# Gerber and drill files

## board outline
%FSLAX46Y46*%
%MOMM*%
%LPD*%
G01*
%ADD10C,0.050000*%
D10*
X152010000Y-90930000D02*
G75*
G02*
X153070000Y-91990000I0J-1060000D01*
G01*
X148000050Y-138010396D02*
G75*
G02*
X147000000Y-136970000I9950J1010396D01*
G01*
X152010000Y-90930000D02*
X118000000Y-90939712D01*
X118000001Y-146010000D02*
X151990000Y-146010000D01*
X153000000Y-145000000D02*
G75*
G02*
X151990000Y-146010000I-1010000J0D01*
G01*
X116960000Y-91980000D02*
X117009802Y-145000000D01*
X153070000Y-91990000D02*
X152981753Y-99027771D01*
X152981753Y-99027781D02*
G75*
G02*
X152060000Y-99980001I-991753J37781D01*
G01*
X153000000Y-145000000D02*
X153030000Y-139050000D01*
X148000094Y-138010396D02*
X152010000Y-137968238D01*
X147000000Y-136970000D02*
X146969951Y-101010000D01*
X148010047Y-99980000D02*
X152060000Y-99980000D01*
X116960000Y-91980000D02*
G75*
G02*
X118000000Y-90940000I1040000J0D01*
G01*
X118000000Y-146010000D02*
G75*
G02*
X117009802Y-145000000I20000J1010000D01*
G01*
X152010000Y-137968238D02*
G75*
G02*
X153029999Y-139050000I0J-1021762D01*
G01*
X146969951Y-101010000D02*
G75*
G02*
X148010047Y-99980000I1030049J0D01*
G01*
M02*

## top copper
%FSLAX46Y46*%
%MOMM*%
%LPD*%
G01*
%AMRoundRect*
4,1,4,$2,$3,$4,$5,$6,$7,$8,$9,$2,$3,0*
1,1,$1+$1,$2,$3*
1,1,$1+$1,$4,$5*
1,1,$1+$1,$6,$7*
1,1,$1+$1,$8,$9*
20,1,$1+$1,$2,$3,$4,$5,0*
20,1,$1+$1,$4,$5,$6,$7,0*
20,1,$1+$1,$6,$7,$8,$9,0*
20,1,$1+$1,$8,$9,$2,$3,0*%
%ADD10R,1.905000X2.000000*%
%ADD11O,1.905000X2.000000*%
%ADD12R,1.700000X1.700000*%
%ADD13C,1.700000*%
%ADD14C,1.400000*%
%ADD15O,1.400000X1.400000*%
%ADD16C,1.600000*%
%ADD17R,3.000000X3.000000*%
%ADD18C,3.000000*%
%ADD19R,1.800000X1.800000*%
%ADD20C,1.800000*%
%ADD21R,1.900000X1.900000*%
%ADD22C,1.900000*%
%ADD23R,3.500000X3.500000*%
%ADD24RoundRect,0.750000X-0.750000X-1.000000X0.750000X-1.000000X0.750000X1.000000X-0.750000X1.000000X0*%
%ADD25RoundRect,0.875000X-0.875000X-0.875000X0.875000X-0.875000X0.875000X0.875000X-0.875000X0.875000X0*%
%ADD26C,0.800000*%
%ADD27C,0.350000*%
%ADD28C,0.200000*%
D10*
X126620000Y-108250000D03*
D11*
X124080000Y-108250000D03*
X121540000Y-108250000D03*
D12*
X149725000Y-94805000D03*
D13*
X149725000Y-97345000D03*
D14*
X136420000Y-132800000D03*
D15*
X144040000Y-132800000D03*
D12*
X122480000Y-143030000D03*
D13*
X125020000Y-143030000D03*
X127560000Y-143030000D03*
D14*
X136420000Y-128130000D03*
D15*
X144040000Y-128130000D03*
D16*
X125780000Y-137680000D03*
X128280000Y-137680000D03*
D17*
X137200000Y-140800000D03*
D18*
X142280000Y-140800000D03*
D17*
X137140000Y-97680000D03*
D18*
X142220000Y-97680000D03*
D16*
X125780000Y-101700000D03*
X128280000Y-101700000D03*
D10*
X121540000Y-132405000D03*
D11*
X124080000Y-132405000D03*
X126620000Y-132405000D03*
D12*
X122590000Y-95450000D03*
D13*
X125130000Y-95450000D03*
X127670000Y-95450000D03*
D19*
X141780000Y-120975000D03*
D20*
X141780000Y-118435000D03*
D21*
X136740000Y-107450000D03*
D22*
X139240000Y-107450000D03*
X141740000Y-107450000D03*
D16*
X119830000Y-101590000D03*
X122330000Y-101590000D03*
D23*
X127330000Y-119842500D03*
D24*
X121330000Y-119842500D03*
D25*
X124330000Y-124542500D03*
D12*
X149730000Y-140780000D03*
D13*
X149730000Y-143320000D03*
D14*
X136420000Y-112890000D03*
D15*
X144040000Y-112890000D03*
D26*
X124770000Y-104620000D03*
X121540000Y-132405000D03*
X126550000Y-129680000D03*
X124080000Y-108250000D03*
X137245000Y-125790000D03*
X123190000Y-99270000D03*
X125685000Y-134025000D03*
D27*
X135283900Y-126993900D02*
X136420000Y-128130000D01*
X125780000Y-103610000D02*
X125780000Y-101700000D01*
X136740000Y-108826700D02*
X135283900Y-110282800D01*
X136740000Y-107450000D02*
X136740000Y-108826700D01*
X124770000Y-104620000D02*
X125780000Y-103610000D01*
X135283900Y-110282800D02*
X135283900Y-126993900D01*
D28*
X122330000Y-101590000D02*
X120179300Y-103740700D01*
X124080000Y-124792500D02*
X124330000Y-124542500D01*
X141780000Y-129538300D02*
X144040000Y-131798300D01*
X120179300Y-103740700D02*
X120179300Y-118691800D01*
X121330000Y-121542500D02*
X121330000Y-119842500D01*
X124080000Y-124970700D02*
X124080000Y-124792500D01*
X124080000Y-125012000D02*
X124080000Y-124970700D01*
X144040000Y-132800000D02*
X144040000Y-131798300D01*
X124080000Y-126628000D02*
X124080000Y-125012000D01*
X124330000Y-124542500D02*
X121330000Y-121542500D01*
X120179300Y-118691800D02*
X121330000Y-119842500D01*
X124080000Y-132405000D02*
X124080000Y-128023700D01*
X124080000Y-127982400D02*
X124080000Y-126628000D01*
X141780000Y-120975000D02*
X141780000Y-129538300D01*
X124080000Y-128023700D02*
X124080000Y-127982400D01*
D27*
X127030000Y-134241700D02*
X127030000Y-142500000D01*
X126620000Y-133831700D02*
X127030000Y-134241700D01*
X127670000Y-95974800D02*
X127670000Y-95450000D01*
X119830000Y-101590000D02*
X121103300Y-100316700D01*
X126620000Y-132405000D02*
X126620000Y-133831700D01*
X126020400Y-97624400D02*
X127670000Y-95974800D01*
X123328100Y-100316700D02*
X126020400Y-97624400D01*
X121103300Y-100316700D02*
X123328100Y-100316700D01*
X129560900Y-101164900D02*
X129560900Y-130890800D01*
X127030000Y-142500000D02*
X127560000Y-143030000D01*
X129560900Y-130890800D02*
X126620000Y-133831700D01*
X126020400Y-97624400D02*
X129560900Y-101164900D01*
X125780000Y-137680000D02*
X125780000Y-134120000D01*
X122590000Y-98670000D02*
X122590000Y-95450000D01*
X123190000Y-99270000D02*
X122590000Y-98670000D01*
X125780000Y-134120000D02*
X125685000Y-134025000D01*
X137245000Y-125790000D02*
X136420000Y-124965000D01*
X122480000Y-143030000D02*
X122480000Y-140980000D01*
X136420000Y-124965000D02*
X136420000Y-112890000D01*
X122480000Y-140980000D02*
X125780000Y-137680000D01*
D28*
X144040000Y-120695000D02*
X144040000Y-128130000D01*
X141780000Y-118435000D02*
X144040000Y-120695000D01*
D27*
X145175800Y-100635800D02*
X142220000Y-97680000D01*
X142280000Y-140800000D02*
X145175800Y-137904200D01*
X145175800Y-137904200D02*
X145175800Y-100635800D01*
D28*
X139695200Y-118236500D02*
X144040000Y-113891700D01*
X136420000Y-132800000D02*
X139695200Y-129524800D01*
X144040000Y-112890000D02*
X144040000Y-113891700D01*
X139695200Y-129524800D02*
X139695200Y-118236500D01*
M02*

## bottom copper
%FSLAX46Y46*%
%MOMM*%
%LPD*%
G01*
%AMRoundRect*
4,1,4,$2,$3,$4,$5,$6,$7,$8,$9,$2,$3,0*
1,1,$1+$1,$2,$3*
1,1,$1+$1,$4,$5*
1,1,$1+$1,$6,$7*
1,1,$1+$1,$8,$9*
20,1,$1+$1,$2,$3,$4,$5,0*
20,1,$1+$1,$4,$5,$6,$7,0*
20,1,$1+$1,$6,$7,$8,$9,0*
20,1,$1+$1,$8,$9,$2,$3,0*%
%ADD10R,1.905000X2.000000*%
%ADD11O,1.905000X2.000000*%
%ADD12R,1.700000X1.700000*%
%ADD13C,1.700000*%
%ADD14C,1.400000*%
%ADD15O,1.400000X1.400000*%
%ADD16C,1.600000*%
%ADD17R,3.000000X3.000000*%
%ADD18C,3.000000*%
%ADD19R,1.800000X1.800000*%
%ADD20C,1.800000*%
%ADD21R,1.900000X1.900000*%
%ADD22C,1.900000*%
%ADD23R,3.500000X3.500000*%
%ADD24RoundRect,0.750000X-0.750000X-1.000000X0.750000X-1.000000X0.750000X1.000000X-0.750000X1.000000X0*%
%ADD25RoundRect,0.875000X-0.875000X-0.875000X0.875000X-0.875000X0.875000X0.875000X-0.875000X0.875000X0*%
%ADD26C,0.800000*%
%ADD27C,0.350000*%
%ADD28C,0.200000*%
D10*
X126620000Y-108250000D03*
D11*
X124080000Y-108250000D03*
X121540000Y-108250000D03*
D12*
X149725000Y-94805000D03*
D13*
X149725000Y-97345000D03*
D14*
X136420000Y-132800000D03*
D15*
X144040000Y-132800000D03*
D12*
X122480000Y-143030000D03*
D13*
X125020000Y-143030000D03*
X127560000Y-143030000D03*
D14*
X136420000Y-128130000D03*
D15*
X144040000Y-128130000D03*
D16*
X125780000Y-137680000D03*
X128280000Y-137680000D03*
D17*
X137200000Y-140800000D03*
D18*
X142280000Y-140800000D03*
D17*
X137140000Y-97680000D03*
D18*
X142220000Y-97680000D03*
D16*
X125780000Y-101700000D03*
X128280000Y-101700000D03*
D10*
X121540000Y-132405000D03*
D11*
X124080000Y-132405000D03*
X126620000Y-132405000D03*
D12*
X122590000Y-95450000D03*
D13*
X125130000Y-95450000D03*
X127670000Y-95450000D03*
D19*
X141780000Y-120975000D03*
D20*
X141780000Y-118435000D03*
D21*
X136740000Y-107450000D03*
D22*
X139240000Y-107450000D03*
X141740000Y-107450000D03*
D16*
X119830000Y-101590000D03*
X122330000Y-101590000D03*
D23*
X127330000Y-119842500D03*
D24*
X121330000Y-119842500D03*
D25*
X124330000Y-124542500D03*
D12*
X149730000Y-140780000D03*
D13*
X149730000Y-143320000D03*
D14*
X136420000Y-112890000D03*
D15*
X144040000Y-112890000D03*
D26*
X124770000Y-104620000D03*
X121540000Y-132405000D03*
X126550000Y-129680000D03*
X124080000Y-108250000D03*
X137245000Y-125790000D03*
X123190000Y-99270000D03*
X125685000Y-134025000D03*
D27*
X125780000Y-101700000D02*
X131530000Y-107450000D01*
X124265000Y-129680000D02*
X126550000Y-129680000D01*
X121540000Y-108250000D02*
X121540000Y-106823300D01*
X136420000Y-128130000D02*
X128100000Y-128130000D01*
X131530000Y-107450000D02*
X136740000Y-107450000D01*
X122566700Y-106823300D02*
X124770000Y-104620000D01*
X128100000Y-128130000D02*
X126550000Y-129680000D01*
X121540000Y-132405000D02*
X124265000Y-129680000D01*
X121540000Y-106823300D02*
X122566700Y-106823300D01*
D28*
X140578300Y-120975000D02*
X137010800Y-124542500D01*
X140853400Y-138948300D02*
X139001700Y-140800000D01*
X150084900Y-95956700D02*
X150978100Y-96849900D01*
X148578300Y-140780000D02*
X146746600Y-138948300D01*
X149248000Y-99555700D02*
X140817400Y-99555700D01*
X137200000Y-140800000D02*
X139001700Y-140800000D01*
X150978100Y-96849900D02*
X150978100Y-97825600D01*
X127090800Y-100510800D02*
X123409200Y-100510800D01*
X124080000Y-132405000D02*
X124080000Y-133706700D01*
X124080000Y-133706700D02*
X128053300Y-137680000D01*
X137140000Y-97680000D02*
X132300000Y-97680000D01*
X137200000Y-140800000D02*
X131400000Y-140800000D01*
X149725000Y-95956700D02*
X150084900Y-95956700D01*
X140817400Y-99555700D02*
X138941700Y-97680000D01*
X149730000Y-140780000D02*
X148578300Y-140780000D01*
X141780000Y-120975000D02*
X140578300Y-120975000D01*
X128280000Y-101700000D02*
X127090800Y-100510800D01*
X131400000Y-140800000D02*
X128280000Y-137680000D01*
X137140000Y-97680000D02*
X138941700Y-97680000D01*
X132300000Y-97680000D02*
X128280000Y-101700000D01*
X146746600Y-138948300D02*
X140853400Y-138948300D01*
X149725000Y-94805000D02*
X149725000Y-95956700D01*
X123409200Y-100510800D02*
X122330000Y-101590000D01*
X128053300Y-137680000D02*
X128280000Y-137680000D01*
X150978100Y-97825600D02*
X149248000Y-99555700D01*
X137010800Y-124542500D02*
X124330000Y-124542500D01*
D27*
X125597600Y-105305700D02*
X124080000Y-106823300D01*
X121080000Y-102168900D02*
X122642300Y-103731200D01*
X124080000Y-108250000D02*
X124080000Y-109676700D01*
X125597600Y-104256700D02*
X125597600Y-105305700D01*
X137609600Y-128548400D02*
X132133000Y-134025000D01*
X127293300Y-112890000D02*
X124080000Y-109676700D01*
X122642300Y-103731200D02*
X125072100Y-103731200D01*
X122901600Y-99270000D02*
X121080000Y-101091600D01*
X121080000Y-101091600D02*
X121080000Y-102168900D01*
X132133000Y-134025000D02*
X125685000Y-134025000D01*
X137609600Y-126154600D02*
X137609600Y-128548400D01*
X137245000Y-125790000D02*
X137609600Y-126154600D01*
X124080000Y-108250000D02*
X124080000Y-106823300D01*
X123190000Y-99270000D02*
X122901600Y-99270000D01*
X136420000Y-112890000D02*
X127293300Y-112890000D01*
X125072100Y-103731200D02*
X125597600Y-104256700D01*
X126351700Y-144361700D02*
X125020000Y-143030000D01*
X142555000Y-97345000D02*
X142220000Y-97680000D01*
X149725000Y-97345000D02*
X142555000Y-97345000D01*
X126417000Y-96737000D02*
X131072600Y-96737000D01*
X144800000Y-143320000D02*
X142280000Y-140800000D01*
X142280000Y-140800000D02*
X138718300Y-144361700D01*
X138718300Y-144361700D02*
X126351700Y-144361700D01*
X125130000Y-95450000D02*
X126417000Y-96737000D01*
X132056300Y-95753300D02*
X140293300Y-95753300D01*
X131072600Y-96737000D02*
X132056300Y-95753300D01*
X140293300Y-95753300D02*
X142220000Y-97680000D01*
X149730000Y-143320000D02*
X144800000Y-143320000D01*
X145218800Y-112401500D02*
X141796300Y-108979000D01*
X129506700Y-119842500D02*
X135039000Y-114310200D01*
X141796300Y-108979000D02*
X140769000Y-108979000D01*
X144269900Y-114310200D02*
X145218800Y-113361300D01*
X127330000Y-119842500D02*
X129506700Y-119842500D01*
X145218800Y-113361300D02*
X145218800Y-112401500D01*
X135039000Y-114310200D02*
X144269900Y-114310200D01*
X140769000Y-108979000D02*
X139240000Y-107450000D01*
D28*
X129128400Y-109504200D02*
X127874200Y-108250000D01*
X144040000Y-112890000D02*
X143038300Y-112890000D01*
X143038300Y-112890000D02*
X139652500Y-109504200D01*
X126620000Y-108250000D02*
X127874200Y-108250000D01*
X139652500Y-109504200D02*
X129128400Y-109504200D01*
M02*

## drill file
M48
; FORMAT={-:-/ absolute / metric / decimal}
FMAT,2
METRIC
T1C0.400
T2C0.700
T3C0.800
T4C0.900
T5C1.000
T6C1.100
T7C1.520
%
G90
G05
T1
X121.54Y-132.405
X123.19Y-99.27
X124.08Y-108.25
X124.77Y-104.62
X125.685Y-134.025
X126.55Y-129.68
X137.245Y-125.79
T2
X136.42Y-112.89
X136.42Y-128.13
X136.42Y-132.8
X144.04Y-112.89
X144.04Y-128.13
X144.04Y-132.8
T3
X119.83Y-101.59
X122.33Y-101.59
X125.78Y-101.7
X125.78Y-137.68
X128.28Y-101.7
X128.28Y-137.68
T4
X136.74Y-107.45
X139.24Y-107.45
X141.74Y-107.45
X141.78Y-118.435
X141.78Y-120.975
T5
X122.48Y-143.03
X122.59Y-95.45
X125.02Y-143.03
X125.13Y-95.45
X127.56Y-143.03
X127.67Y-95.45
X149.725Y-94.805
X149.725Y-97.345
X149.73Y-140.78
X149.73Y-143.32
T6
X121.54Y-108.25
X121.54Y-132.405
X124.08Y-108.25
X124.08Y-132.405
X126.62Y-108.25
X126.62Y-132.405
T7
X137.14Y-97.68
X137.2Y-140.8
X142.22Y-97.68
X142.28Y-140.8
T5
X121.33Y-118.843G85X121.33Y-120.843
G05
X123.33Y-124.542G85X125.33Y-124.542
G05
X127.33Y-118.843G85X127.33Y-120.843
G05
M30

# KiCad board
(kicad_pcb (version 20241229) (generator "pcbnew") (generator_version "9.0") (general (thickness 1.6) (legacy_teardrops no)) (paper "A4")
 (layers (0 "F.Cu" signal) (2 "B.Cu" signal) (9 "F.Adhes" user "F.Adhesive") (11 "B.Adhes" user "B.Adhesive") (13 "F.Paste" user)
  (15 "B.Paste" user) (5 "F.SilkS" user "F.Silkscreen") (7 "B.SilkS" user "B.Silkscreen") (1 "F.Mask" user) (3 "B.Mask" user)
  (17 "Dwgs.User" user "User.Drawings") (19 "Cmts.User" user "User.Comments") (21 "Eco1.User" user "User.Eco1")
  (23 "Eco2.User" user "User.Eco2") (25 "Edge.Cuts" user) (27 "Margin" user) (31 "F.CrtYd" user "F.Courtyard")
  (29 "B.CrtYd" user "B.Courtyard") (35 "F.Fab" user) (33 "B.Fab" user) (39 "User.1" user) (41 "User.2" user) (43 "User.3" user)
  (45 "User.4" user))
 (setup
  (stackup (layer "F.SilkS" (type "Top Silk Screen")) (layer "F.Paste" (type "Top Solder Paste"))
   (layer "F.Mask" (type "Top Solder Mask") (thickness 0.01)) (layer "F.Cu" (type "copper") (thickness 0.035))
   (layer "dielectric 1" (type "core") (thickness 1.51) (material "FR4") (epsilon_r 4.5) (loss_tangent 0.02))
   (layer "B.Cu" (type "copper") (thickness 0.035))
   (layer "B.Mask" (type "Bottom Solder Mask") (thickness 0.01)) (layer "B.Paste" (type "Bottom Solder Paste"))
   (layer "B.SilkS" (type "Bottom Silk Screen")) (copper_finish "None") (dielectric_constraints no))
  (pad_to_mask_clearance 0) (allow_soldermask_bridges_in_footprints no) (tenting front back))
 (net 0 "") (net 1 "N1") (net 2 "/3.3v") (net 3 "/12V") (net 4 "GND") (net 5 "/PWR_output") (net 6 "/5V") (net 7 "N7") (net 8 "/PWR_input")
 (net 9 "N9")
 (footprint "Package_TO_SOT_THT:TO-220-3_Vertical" (layer "F.Cu") (at 126.62 108.25 180)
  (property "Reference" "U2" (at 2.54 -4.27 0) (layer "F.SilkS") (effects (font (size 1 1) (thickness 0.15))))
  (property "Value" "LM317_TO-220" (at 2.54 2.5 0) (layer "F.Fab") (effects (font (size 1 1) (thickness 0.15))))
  (pad "1" thru_hole rect (at 0 0 180) (size 1.905 2) (drill 1.1) (layers "*.Cu" "*.Mask") (remove_unused_layers no) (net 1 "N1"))
  (pad "2" thru_hole oval (at 2.54 0 180) (size 1.905 2) (drill 1.1) (layers "*.Cu" "*.Mask") (remove_unused_layers no) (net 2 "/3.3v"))
  (pad "3" thru_hole oval (at 5.08 0 180) (size 1.905 2) (drill 1.1) (layers "*.Cu" "*.Mask") (remove_unused_layers no) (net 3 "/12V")))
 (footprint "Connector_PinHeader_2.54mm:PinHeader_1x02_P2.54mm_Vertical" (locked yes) (layer "F.Cu") (at 149.725 94.805)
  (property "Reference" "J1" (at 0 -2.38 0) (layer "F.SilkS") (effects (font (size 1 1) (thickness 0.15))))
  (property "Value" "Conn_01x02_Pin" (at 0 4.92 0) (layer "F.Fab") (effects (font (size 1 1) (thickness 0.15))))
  (pad "1" thru_hole rect (at 0 0) (size 1.7 1.7) (drill 1) (layers "*.Cu" "*.Mask") (remove_unused_layers no) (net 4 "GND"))
  (pad "2" thru_hole circle (at 0 2.54) (size 1.7 1.7) (drill 1) (layers "*.Cu" "*.Mask") (remove_unused_layers no) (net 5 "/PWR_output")))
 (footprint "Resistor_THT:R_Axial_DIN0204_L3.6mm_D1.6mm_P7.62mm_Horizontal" (layer "F.Cu") (at 136.42 132.8)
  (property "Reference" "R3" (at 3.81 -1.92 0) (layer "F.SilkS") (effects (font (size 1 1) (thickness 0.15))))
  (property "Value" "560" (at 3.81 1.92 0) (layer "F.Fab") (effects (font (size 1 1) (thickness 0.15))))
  (pad "1" thru_hole circle (at 0 0) (size 1.4 1.4) (drill 0.7) (layers "*.Cu" "*.Mask") (remove_unused_layers no) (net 1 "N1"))
  (pad "2" thru_hole oval (at 7.62 0) (size 1.4 1.4) (drill 0.7) (layers "*.Cu" "*.Mask") (remove_unused_layers no) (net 4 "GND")))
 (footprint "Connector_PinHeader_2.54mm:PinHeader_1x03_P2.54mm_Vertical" (layer "F.Cu") (at 122.48 143.03 90)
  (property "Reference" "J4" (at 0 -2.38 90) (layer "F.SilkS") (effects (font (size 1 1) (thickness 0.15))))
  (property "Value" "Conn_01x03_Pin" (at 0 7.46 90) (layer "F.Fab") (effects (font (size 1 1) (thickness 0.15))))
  (pad "1" thru_hole rect (at 0 0 90) (size 1.7 1.7) (drill 1) (layers "*.Cu" "*.Mask") (remove_unused_layers no) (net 2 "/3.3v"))
  (pad "2" thru_hole circle (at 0 2.54 90) (size 1.7 1.7) (drill 1) (layers "*.Cu" "*.Mask") (remove_unused_layers no) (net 5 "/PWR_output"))
  (pad "3" thru_hole circle (at 0 5.08 90) (size 1.7 1.7) (drill 1) (layers "*.Cu" "*.Mask") (remove_unused_layers no) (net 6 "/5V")))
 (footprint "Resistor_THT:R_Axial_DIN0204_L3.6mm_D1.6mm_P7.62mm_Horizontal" (layer "F.Cu") (at 136.42 128.13)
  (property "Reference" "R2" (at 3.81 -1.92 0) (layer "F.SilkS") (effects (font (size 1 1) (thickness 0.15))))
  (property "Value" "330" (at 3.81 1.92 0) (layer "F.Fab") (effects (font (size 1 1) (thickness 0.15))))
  (pad "1" thru_hole circle (at 0 0) (size 1.4 1.4) (drill 0.7) (layers "*.Cu" "*.Mask") (remove_unused_layers no) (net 3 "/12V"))
  (pad "2" thru_hole oval (at 7.62 0) (size 1.4 1.4) (drill 0.7) (layers "*.Cu" "*.Mask") (remove_unused_layers no) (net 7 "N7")))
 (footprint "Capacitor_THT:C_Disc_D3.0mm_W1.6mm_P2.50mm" (layer "F.Cu") (at 125.78 137.68)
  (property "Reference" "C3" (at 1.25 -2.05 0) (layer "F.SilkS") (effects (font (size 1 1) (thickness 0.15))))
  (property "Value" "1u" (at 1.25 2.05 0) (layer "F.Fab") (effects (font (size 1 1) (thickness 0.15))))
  (pad "1" thru_hole circle (at 0 0) (size 1.6 1.6) (drill 0.8) (layers "*.Cu" "*.Mask") (remove_unused_layers no) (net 2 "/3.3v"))
  (pad "2" thru_hole circle (at 2.5 0) (size 1.6 1.6) (drill 0.8) (layers "*.Cu" "*.Mask") (remove_unused_layers no) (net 4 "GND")))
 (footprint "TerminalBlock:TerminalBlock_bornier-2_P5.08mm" (layer "F.Cu") (at 137.2 140.8)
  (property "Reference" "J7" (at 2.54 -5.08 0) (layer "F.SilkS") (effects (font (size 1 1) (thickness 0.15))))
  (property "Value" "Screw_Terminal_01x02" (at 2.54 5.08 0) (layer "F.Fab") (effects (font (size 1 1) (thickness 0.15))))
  (pad "1" thru_hole rect (at 0 0) (size 3 3) (drill 1.52) (layers "*.Cu" "*.Mask") (remove_unused_layers no) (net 4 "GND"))
  (pad "2" thru_hole circle (at 5.08 0) (size 3 3) (drill 1.52) (layers "*.Cu" "*.Mask") (remove_unused_layers no) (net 5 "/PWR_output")))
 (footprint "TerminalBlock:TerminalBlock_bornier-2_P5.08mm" (layer "F.Cu") (at 137.14 97.68)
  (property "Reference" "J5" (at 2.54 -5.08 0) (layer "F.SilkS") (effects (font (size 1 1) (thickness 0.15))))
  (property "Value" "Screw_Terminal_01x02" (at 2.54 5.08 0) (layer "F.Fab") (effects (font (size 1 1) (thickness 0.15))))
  (pad "1" thru_hole rect (at 0 0) (size 3 3) (drill 1.52) (layers "*.Cu" "*.Mask") (remove_unused_layers no) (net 4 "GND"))
  (pad "2" thru_hole circle (at 5.08 0) (size 3 3) (drill 1.52) (layers "*.Cu" "*.Mask") (remove_unused_layers no) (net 5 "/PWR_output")))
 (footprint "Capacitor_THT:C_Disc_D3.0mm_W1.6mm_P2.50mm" (layer "F.Cu") (at 125.78 101.7)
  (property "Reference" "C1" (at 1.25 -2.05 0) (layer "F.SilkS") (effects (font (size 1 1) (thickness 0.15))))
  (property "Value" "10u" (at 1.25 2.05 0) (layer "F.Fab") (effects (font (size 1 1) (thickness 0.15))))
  (pad "1" thru_hole circle (at 0 0) (size 1.6 1.6) (drill 0.8) (layers "*.Cu" "*.Mask") (remove_unused_layers no) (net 3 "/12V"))
  (pad "2" thru_hole circle (at 2.5 0) (size 1.6 1.6) (drill 0.8) (layers "*.Cu" "*.Mask") (remove_unused_layers no) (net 4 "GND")))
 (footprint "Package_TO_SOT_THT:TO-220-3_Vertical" (layer "F.Cu") (at 121.54 132.405)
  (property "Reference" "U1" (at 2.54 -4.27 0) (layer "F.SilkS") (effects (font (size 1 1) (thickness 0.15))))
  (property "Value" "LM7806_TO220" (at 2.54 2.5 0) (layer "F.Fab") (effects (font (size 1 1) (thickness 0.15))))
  (pad "1" thru_hole rect (at 0 0) (size 1.905 2) (drill 1.1) (layers "*.Cu" "*.Mask") (remove_unused_layers no) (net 3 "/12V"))
  (pad "2" thru_hole oval (at 2.54 0) (size 1.905 2) (drill 1.1) (layers "*.Cu" "*.Mask") (remove_unused_layers no) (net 4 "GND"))
  (pad "3" thru_hole oval (at 5.08 0) (size 1.905 2) (drill 1.1) (layers "*.Cu" "*.Mask") (remove_unused_layers no) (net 6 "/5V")))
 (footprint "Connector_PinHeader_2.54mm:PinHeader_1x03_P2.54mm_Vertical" (layer "F.Cu") (at 122.59 95.45 90)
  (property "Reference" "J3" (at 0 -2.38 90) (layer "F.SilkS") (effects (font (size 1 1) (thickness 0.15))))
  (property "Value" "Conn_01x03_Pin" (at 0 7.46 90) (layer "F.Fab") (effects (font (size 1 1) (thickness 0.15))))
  (pad "1" thru_hole rect (at 0 0 90) (size 1.7 1.7) (drill 1) (layers "*.Cu" "*.Mask") (remove_unused_layers no) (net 2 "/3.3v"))
  (pad "2" thru_hole circle (at 0 2.54 90) (size 1.7 1.7) (drill 1) (layers "*.Cu" "*.Mask") (remove_unused_layers no) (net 5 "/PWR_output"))
  (pad "3" thru_hole circle (at 0 5.08 90) (size 1.7 1.7) (drill 1) (layers "*.Cu" "*.Mask") (remove_unused_layers no) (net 6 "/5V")))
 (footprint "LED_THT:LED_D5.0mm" (layer "F.Cu") (at 141.78 120.975 90)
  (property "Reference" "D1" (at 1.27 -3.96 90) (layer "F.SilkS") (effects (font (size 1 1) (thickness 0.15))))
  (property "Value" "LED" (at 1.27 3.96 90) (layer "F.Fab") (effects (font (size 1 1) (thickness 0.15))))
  (pad "1" thru_hole rect (at 0 0 90) (size 1.8 1.8) (drill 0.9) (layers "*.Cu" "*.Mask") (remove_unused_layers no) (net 4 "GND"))
  (pad "2" thru_hole circle (at 2.54 0 90) (size 1.8 1.8) (drill 0.9) (layers "*.Cu" "*.Mask") (remove_unused_layers no) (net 7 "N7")))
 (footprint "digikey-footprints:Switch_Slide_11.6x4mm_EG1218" (layer "F.Cu") (at 136.74 107.45)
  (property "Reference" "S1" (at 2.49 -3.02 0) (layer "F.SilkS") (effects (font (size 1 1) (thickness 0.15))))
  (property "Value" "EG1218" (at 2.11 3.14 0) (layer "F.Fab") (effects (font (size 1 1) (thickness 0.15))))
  (pad "1" thru_hole rect (at 0 0) (size 1.9 1.9) (drill 0.9) (layers "*.Cu" "*.Mask") (remove_unused_layers no) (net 3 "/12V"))
  (pad "2" thru_hole circle (at 2.5 0) (size 1.9 1.9) (drill 0.9) (layers "*.Cu" "*.Mask") (remove_unused_layers no) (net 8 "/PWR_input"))
  (pad "3" thru_hole circle (at 5 0) (size 1.9 1.9) (drill 0.9) (layers "*.Cu" "*.Mask") (remove_unused_layers no) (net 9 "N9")))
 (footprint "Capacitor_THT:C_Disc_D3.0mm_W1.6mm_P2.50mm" (layer "F.Cu") (at 119.83 101.59)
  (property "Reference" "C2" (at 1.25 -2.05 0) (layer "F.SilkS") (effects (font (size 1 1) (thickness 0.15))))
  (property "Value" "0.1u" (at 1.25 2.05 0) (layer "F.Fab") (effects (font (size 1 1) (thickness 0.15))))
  (pad "1" thru_hole circle (at 0 0) (size 1.6 1.6) (drill 0.8) (layers "*.Cu" "*.Mask") (remove_unused_layers no) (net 6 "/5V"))
  (pad "2" thru_hole circle (at 2.5 0) (size 1.6 1.6) (drill 0.8) (layers "*.Cu" "*.Mask") (remove_unused_layers no) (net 4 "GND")))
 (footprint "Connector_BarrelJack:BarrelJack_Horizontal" (layer "F.Cu") (at 127.33 119.8425)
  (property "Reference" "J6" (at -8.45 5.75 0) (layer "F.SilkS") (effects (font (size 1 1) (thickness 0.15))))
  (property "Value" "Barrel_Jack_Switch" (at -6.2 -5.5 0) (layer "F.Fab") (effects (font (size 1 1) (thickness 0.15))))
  (pad "1" thru_hole rect (at 0 0) (size 3.5 3.5) (drill oval 1 3) (layers "*.Cu" "*.Mask") (remove_unused_layers no) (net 8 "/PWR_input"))
  (pad "2" thru_hole roundrect (at -6 0) (size 3 3.5) (drill oval 1 3) (layers "*.Cu" "*.Mask") (remove_unused_layers no)
   (roundrect_rratio 0.25) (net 4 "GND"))
  (pad "3" thru_hole roundrect (at -3 4.7) (size 3.5 3.5) (drill oval 3 1) (layers "*.Cu" "*.Mask") (remove_unused_layers no)
   (roundrect_rratio 0.25) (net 4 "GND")))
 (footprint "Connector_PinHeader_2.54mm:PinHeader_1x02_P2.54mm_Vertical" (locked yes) (layer "F.Cu") (at 149.73 140.78)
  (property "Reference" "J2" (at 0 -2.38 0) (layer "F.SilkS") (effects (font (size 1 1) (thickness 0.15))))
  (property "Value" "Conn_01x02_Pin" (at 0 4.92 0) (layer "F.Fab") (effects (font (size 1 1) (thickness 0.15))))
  (pad "1" thru_hole rect (at 0 0) (size 1.7 1.7) (drill 1) (layers "*.Cu" "*.Mask") (remove_unused_layers no) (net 4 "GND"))
  (pad "2" thru_hole circle (at 0 2.54) (size 1.7 1.7) (drill 1) (layers "*.Cu" "*.Mask") (remove_unused_layers no) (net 5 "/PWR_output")))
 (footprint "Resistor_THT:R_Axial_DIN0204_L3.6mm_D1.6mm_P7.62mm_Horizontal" (layer "F.Cu") (at 136.42 112.89)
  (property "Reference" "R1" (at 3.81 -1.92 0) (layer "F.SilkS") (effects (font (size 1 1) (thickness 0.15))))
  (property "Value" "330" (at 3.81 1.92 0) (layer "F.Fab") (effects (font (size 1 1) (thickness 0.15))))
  (pad "1" thru_hole circle (at 0 0) (size 1.4 1.4) (drill 0.7) (layers "*.Cu" "*.Mask") (remove_unused_layers no) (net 2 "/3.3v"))
  (pad "2" thru_hole oval (at 7.62 0) (size 1.4 1.4) (drill 0.7) (layers "*.Cu" "*.Mask") (remove_unused_layers no) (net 1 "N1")))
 (gr_arc (start 152.01 90.93) (mid 152.759533 91.240467) (end 153.07 91.99) (stroke (width 0.05) (type default)) (layer "Edge.Cuts"))
 (gr_arc (start 148.00005 138.010396) (mid 147.281522 137.700228) (end 147 136.97) (stroke (width 0.05) (type default)) (layer "Edge.Cuts"))
 (gr_line (start 152.01 90.93) (end 118 90.939712) (stroke (width 0.05) (type default)) (layer "Edge.Cuts"))
 (gr_line (start 118.000001 146.01) (end 151.99 146.01) (stroke (width 0.05) (type default)) (layer "Edge.Cuts"))
 (gr_arc (start 153 145) (mid 152.704178 145.714178) (end 151.99 146.01) (stroke (width 0.05) (type default)) (layer "Edge.Cuts"))
 (gr_line (start 116.96 91.98) (end 117.009802 145) (stroke (width 0.05) (type default)) (layer "Edge.Cuts"))
 (gr_line (start 153.07 91.99) (end 152.981753 99.027771) (stroke (width 0.05) (type default)) (layer "Edge.Cuts"))
 (gr_arc (start 152.981753 99.027781) (mid 152.703099 99.680283) (end 152.06 99.98) (stroke (width 0.05) (type default)) (layer "Edge.Cuts"))
 (gr_line (start 153 145) (end 153.03 139.05) (stroke (width 0.05) (type default)) (layer "Edge.Cuts"))
 (gr_line (start 148.000094 138.010396) (end 152.01 137.968238) (stroke (width 0.05) (type default)) (layer "Edge.Cuts"))
 (gr_line (start 147 136.97) (end 146.969951 101.01) (stroke (width 0.05) (type default)) (layer "Edge.Cuts"))
 (gr_line (start 148.010047 99.98) (end 152.06 99.98) (stroke (width 0.05) (type solid)) (layer "Edge.Cuts"))
 (gr_arc (start 116.96 91.98) (mid 117.264609 91.244609) (end 118 90.94) (stroke (width 0.05) (type default)) (layer "Edge.Cuts"))
 (gr_arc (start 118 146.01) (mid 117.298646 145.707211) (end 117.009802 145) (stroke (width 0.05) (type default)) (layer "Edge.Cuts"))
 (gr_arc (start 152.01 137.968238) (mid 152.753405 138.289039) (end 153.029999 139.05) (stroke (width 0.05) (type default))
  (layer "Edge.Cuts"))
 (gr_arc (start 146.969951 101.01) (mid 147.275206 100.278102) (end 148.010047 99.98) (stroke (width 0.05) (type default))
  (layer "Edge.Cuts"))
 (segment (start 135.2839 126.9939) (end 136.42 128.13) (width 0.35) (layer "F.Cu") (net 3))
 (segment (start 125.78 103.61) (end 125.78 101.7) (width 0.35) (layer "F.Cu") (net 3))
 (segment (start 136.74 108.8267) (end 135.2839 110.2828) (width 0.35) (layer "F.Cu") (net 3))
 (segment (start 136.74 107.45) (end 136.74 108.8267) (width 0.35) (layer "F.Cu") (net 3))
 (segment (start 124.77 104.62) (end 125.78 103.61) (width 0.35) (layer "F.Cu") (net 3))
 (segment (start 135.2839 110.2828) (end 135.2839 126.9939) (width 0.35) (layer "F.Cu") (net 3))
 (via (at 124.77 104.62) (size 0.8) (drill 0.4) (layers "F.Cu" "B.Cu") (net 3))
 (via (at 121.54 132.405) (size 0.8) (drill 0.4) (layers "F.Cu" "B.Cu") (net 3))
 (via (at 126.55 129.68) (size 0.8) (drill 0.4) (layers "F.Cu" "B.Cu") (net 3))
 (segment (start 125.78 101.7) (end 131.53 107.45) (width 0.35) (layer "B.Cu") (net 3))
 (segment (start 124.265 129.68) (end 126.55 129.68) (width 0.35) (layer "B.Cu") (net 3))
 (segment (start 121.54 108.25) (end 121.54 106.8233) (width 0.35) (layer "B.Cu") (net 3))
 (segment (start 136.42 128.13) (end 128.1 128.13) (width 0.35) (layer "B.Cu") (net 3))
 (segment (start 131.53 107.45) (end 136.74 107.45) (width 0.35) (layer "B.Cu") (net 3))
 (segment (start 122.5667 106.8233) (end 124.77 104.62) (width 0.35) (layer "B.Cu") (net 3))
 (segment (start 128.1 128.13) (end 126.55 129.68) (width 0.35) (layer "B.Cu") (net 3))
 (segment (start 121.54 132.405) (end 124.265 129.68) (width 0.35) (layer "B.Cu") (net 3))
 (segment (start 121.54 106.8233) (end 122.5667 106.8233) (width 0.35) (layer "B.Cu") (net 3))
 (segment (start 122.33 101.59) (end 120.1793 103.7407) (width 0.2) (layer "F.Cu") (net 4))
 (segment (start 124.08 124.7925) (end 124.33 124.5425) (width 0.2) (layer "F.Cu") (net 4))
 (segment (start 141.78 129.5383) (end 144.04 131.7983) (width 0.2) (layer "F.Cu") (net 4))
 (segment (start 120.1793 103.7407) (end 120.1793 118.6918) (width 0.2) (layer "F.Cu") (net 4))
 (segment (start 121.33 121.5425) (end 121.33 119.8425) (width 0.2) (layer "F.Cu") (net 4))
 (segment (start 124.08 124.9707) (end 124.08 124.7925) (width 0.2) (layer "F.Cu") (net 4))
 (segment (start 124.08 125.012) (end 124.08 124.9707) (width 0.2) (layer "F.Cu") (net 4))
 (segment (start 144.04 132.8) (end 144.04 131.7983) (width 0.2) (layer "F.Cu") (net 4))
 (segment (start 124.08 126.628) (end 124.08 125.012) (width 0.2) (layer "F.Cu") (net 4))
 (segment (start 124.33 124.5425) (end 121.33 121.5425) (width 0.2) (layer "F.Cu") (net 4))
 (segment (start 120.1793 118.6918) (end 121.33 119.8425) (width 0.2) (layer "F.Cu") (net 4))
 (segment (start 124.08 132.405) (end 124.08 128.0237) (width 0.2) (layer "F.Cu") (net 4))
 (segment (start 124.08 127.9824) (end 124.08 126.628) (width 0.2) (layer "F.Cu") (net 4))
 (segment (start 141.78 120.975) (end 141.78 129.5383) (width 0.2) (layer "F.Cu") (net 4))
 (segment (start 124.08 128.0237) (end 124.08 127.9824) (width 0.2) (layer "F.Cu") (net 4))
 (segment (start 140.5783 120.975) (end 137.0108 124.5425) (width 0.2) (layer "B.Cu") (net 4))
 (segment (start 140.8534 138.9483) (end 139.0017 140.8) (width 0.2) (layer "B.Cu") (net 4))
 (segment (start 150.0849 95.9567) (end 150.9781 96.8499) (width 0.2) (layer "B.Cu") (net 4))
 (segment (start 148.5783 140.78) (end 146.7466 138.9483) (width 0.2) (layer "B.Cu") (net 4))
 (segment (start 149.248 99.5557) (end 140.8174 99.5557) (width 0.2) (layer "B.Cu") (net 4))
 (segment (start 137.2 140.8) (end 139.0017 140.8) (width 0.2) (layer "B.Cu") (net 4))
 (segment (start 150.9781 96.8499) (end 150.9781 97.8256) (width 0.2) (layer "B.Cu") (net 4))
 (segment (start 127.0908 100.5108) (end 123.4092 100.5108) (width 0.2) (layer "B.Cu") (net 4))
 (segment (start 124.08 132.405) (end 124.08 133.7067) (width 0.2) (layer "B.Cu") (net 4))
 (segment (start 124.08 133.7067) (end 128.0533 137.68) (width 0.2) (layer "B.Cu") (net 4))
 (segment (start 137.14 97.68) (end 132.3 97.68) (width 0.2) (layer "B.Cu") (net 4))
 (segment (start 137.2 140.8) (end 131.4 140.8) (width 0.2) (layer "B.Cu") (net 4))
 (segment (start 149.725 95.9567) (end 150.0849 95.9567) (width 0.2) (layer "B.Cu") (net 4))
 (segment (start 140.8174 99.5557) (end 138.9417 97.68) (width 0.2) (layer "B.Cu") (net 4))
 (segment (start 149.73 140.78) (end 148.5783 140.78) (width 0.2) (layer "B.Cu") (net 4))
 (segment (start 141.78 120.975) (end 140.5783 120.975) (width 0.2) (layer "B.Cu") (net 4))
 (segment (start 128.28 101.7) (end 127.0908 100.5108) (width 0.2) (layer "B.Cu") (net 4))
 (segment (start 131.4 140.8) (end 128.28 137.68) (width 0.2) (layer "B.Cu") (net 4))
 (segment (start 137.14 97.68) (end 138.9417 97.68) (width 0.2) (layer "B.Cu") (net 4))
 (segment (start 132.3 97.68) (end 128.28 101.7) (width 0.2) (layer "B.Cu") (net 4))
 (segment (start 146.7466 138.9483) (end 140.8534 138.9483) (width 0.2) (layer "B.Cu") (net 4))
 (segment (start 149.725 94.805) (end 149.725 95.9567) (width 0.2) (layer "B.Cu") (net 4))
 (segment (start 123.4092 100.5108) (end 122.33 101.59) (width 0.2) (layer "B.Cu") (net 4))
 (segment (start 128.0533 137.68) (end 128.28 137.68) (width 0.2) (layer "B.Cu") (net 4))
 (segment (start 150.9781 97.8256) (end 149.248 99.5557) (width 0.2) (layer "B.Cu") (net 4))
 (segment (start 137.0108 124.5425) (end 124.33 124.5425) (width 0.2) (layer "B.Cu") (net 4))
 (segment (start 127.03 134.2417) (end 127.03 142.5) (width 0.35) (layer "F.Cu") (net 6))
 (segment (start 126.62 133.8317) (end 127.03 134.2417) (width 0.35) (layer "F.Cu") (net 6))
 (segment (start 127.67 95.9748) (end 127.67 95.45) (width 0.35) (layer "F.Cu") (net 6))
 (segment (start 119.83 101.59) (end 121.1033 100.3167) (width 0.35) (layer "F.Cu") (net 6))
 (segment (start 126.62 132.405) (end 126.62 133.8317) (width 0.35) (layer "F.Cu") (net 6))
 (segment (start 126.0204 97.6244) (end 127.67 95.9748) (width 0.35) (layer "F.Cu") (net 6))
 (segment (start 123.3281 100.3167) (end 126.0204 97.6244) (width 0.35) (layer "F.Cu") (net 6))
 (segment (start 121.1033 100.3167) (end 123.3281 100.3167) (width 0.35) (layer "F.Cu") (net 6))
 (segment (start 129.5609 101.1649) (end 129.5609 130.8908) (width 0.35) (layer "F.Cu") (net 6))
 (segment (start 127.03 142.5) (end 127.56 143.03) (width 0.35) (layer "F.Cu") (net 6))
 (segment (start 129.5609 130.8908) (end 126.62 133.8317) (width 0.35) (layer "F.Cu") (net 6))
 (segment (start 126.0204 97.6244) (end 129.5609 101.1649) (width 0.35) (layer "F.Cu") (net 6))
 (segment (start 125.78 137.68) (end 125.78 134.12) (width 0.35) (layer "F.Cu") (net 2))
 (segment (start 122.59 98.67) (end 122.59 95.45) (width 0.35) (layer "F.Cu") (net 2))
 (segment (start 123.19 99.27) (end 122.59 98.67) (width 0.35) (layer "F.Cu") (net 2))
 (segment (start 125.78 134.12) (end 125.685 134.025) (width 0.35) (layer "F.Cu") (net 2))
 (segment (start 137.245 125.79) (end 136.42 124.965) (width 0.35) (layer "F.Cu") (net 2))
 (segment (start 122.48 143.03) (end 122.48 140.98) (width 0.35) (layer "F.Cu") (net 2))
 (segment (start 136.42 124.965) (end 136.42 112.89) (width 0.35) (layer "F.Cu") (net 2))
 (segment (start 122.48 140.98) (end 125.78 137.68) (width 0.35) (layer "F.Cu") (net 2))
 (via (at 124.08 108.25) (size 0.8) (drill 0.4) (layers "F.Cu" "B.Cu") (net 2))
 (via (at 137.245 125.79) (size 0.8) (drill 0.4) (layers "F.Cu" "B.Cu") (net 2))
 (via (at 123.19 99.27) (size 0.8) (drill 0.4) (layers "F.Cu" "B.Cu") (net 2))
 (via (at 125.685 134.025) (size 0.8) (drill 0.4) (layers "F.Cu" "B.Cu") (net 2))
 (segment (start 125.5976 105.3057) (end 124.08 106.8233) (width 0.35) (layer "B.Cu") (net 2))
 (segment (start 121.08 102.1689) (end 122.6423 103.7312) (width 0.35) (layer "B.Cu") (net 2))
 (segment (start 124.08 108.25) (end 124.08 109.6767) (width 0.35) (layer "B.Cu") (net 2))
 (segment (start 125.5976 104.2567) (end 125.5976 105.3057) (width 0.35) (layer "B.Cu") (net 2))
 (segment (start 137.6096 128.5484) (end 132.133 134.025) (width 0.35) (layer "B.Cu") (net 2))
 (segment (start 127.2933 112.89) (end 124.08 109.6767) (width 0.35) (layer "B.Cu") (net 2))
 (segment (start 122.6423 103.7312) (end 125.0721 103.7312) (width 0.35) (layer "B.Cu") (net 2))
 (segment (start 122.9016 99.27) (end 121.08 101.0916) (width 0.35) (layer "B.Cu") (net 2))
 (segment (start 121.08 101.0916) (end 121.08 102.1689) (width 0.35) (layer "B.Cu") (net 2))
 (segment (start 132.133 134.025) (end 125.685 134.025) (width 0.35) (layer "B.Cu") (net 2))
 (segment (start 137.6096 126.1546) (end 137.6096 128.5484) (width 0.35) (layer "B.Cu") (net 2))
 (segment (start 137.245 125.79) (end 137.6096 126.1546) (width 0.35) (layer "B.Cu") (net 2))
 (segment (start 124.08 108.25) (end 124.08 106.8233) (width 0.35) (layer "B.Cu") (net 2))
 (segment (start 123.19 99.27) (end 122.9016 99.27) (width 0.35) (layer "B.Cu") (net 2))
 (segment (start 136.42 112.89) (end 127.2933 112.89) (width 0.35) (layer "B.Cu") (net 2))
 (segment (start 125.0721 103.7312) (end 125.5976 104.2567) (width 0.35) (layer "B.Cu") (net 2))
 (segment (start 144.04 120.695) (end 144.04 128.13) (width 0.2) (layer "F.Cu") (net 7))
 (segment (start 141.78 118.435) (end 144.04 120.695) (width 0.2) (layer "F.Cu") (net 7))
 (segment (start 145.1758 100.6358) (end 142.22 97.68) (width 0.35) (layer "F.Cu") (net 5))
 (segment (start 142.28 140.8) (end 145.1758 137.9042) (width 0.35) (layer "F.Cu") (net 5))
 (segment (start 145.1758 137.9042) (end 145.1758 100.6358) (width 0.35) (layer "F.Cu") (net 5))
 (segment (start 126.3517 144.3617) (end 125.02 143.03) (width 0.35) (layer "B.Cu") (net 5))
 (segment (start 142.555 97.345) (end 142.22 97.68) (width 0.35) (layer "B.Cu") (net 5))
 (segment (start 149.725 97.345) (end 142.555 97.345) (width 0.35) (layer "B.Cu") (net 5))
 (segment (start 126.417 96.737) (end 131.0726 96.737) (width 0.35) (layer "B.Cu") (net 5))
 (segment (start 144.8 143.32) (end 142.28 140.8) (width 0.35) (layer "B.Cu") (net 5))
 (segment (start 142.28 140.8) (end 138.7183 144.3617) (width 0.35) (layer "B.Cu") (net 5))
 (segment (start 138.7183 144.3617) (end 126.3517 144.3617) (width 0.35) (layer "B.Cu") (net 5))
 (segment (start 125.13 95.45) (end 126.417 96.737) (width 0.35) (layer "B.Cu") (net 5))
 (segment (start 132.0563 95.7533) (end 140.2933 95.7533) (width 0.35) (layer "B.Cu") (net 5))
 (segment (start 131.0726 96.737) (end 132.0563 95.7533) (width 0.35) (layer "B.Cu") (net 5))
 (segment (start 140.2933 95.7533) (end 142.22 97.68) (width 0.35) (layer "B.Cu") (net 5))
 (segment (start 149.73 143.32) (end 144.8 143.32) (width 0.35) (layer "B.Cu") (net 5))
 (segment (start 145.2188 112.4015) (end 141.7963 108.979) (width 0.35) (layer "B.Cu") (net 8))
 (segment (start 129.5067 119.8425) (end 135.039 114.3102) (width 0.35) (layer "B.Cu") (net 8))
 (segment (start 141.7963 108.979) (end 140.769 108.979) (width 0.35) (layer "B.Cu") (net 8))
 (segment (start 144.2699 114.3102) (end 145.2188 113.3613) (width 0.35) (layer "B.Cu") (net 8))
 (segment (start 127.33 119.8425) (end 129.5067 119.8425) (width 0.35) (layer "B.Cu") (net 8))
 (segment (start 145.2188 113.3613) (end 145.2188 112.4015) (width 0.35) (layer "B.Cu") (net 8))
 (segment (start 135.039 114.3102) (end 144.2699 114.3102) (width 0.35) (layer "B.Cu") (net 8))
 (segment (start 140.769 108.979) (end 139.24 107.45) (width 0.35) (layer "B.Cu") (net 8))
 (segment (start 139.6952 118.2365) (end 144.04 113.8917) (width 0.2) (layer "F.Cu") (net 1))
 (segment (start 136.42 132.8) (end 139.6952 129.5248) (width 0.2) (layer "F.Cu") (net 1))
 (segment (start 144.04 112.89) (end 144.04 113.8917) (width 0.2) (layer "F.Cu") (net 1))
 (segment (start 139.6952 129.5248) (end 139.6952 118.2365) (width 0.2) (layer "F.Cu") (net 1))
 (segment (start 129.1284 109.5042) (end 127.8742 108.25) (width 0.2) (layer "B.Cu") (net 1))
 (segment (start 144.04 112.89) (end 143.0383 112.89) (width 0.2) (layer "B.Cu") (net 1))
 (segment (start 143.0383 112.89) (end 139.6525 109.5042) (width 0.2) (layer "B.Cu") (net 1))
 (segment (start 126.62 108.25) (end 127.8742 108.25) (width 0.2) (layer "B.Cu") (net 1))
 (segment (start 139.6525 109.5042) (end 129.1284 109.5042) (width 0.2) (layer "B.Cu") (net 1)))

